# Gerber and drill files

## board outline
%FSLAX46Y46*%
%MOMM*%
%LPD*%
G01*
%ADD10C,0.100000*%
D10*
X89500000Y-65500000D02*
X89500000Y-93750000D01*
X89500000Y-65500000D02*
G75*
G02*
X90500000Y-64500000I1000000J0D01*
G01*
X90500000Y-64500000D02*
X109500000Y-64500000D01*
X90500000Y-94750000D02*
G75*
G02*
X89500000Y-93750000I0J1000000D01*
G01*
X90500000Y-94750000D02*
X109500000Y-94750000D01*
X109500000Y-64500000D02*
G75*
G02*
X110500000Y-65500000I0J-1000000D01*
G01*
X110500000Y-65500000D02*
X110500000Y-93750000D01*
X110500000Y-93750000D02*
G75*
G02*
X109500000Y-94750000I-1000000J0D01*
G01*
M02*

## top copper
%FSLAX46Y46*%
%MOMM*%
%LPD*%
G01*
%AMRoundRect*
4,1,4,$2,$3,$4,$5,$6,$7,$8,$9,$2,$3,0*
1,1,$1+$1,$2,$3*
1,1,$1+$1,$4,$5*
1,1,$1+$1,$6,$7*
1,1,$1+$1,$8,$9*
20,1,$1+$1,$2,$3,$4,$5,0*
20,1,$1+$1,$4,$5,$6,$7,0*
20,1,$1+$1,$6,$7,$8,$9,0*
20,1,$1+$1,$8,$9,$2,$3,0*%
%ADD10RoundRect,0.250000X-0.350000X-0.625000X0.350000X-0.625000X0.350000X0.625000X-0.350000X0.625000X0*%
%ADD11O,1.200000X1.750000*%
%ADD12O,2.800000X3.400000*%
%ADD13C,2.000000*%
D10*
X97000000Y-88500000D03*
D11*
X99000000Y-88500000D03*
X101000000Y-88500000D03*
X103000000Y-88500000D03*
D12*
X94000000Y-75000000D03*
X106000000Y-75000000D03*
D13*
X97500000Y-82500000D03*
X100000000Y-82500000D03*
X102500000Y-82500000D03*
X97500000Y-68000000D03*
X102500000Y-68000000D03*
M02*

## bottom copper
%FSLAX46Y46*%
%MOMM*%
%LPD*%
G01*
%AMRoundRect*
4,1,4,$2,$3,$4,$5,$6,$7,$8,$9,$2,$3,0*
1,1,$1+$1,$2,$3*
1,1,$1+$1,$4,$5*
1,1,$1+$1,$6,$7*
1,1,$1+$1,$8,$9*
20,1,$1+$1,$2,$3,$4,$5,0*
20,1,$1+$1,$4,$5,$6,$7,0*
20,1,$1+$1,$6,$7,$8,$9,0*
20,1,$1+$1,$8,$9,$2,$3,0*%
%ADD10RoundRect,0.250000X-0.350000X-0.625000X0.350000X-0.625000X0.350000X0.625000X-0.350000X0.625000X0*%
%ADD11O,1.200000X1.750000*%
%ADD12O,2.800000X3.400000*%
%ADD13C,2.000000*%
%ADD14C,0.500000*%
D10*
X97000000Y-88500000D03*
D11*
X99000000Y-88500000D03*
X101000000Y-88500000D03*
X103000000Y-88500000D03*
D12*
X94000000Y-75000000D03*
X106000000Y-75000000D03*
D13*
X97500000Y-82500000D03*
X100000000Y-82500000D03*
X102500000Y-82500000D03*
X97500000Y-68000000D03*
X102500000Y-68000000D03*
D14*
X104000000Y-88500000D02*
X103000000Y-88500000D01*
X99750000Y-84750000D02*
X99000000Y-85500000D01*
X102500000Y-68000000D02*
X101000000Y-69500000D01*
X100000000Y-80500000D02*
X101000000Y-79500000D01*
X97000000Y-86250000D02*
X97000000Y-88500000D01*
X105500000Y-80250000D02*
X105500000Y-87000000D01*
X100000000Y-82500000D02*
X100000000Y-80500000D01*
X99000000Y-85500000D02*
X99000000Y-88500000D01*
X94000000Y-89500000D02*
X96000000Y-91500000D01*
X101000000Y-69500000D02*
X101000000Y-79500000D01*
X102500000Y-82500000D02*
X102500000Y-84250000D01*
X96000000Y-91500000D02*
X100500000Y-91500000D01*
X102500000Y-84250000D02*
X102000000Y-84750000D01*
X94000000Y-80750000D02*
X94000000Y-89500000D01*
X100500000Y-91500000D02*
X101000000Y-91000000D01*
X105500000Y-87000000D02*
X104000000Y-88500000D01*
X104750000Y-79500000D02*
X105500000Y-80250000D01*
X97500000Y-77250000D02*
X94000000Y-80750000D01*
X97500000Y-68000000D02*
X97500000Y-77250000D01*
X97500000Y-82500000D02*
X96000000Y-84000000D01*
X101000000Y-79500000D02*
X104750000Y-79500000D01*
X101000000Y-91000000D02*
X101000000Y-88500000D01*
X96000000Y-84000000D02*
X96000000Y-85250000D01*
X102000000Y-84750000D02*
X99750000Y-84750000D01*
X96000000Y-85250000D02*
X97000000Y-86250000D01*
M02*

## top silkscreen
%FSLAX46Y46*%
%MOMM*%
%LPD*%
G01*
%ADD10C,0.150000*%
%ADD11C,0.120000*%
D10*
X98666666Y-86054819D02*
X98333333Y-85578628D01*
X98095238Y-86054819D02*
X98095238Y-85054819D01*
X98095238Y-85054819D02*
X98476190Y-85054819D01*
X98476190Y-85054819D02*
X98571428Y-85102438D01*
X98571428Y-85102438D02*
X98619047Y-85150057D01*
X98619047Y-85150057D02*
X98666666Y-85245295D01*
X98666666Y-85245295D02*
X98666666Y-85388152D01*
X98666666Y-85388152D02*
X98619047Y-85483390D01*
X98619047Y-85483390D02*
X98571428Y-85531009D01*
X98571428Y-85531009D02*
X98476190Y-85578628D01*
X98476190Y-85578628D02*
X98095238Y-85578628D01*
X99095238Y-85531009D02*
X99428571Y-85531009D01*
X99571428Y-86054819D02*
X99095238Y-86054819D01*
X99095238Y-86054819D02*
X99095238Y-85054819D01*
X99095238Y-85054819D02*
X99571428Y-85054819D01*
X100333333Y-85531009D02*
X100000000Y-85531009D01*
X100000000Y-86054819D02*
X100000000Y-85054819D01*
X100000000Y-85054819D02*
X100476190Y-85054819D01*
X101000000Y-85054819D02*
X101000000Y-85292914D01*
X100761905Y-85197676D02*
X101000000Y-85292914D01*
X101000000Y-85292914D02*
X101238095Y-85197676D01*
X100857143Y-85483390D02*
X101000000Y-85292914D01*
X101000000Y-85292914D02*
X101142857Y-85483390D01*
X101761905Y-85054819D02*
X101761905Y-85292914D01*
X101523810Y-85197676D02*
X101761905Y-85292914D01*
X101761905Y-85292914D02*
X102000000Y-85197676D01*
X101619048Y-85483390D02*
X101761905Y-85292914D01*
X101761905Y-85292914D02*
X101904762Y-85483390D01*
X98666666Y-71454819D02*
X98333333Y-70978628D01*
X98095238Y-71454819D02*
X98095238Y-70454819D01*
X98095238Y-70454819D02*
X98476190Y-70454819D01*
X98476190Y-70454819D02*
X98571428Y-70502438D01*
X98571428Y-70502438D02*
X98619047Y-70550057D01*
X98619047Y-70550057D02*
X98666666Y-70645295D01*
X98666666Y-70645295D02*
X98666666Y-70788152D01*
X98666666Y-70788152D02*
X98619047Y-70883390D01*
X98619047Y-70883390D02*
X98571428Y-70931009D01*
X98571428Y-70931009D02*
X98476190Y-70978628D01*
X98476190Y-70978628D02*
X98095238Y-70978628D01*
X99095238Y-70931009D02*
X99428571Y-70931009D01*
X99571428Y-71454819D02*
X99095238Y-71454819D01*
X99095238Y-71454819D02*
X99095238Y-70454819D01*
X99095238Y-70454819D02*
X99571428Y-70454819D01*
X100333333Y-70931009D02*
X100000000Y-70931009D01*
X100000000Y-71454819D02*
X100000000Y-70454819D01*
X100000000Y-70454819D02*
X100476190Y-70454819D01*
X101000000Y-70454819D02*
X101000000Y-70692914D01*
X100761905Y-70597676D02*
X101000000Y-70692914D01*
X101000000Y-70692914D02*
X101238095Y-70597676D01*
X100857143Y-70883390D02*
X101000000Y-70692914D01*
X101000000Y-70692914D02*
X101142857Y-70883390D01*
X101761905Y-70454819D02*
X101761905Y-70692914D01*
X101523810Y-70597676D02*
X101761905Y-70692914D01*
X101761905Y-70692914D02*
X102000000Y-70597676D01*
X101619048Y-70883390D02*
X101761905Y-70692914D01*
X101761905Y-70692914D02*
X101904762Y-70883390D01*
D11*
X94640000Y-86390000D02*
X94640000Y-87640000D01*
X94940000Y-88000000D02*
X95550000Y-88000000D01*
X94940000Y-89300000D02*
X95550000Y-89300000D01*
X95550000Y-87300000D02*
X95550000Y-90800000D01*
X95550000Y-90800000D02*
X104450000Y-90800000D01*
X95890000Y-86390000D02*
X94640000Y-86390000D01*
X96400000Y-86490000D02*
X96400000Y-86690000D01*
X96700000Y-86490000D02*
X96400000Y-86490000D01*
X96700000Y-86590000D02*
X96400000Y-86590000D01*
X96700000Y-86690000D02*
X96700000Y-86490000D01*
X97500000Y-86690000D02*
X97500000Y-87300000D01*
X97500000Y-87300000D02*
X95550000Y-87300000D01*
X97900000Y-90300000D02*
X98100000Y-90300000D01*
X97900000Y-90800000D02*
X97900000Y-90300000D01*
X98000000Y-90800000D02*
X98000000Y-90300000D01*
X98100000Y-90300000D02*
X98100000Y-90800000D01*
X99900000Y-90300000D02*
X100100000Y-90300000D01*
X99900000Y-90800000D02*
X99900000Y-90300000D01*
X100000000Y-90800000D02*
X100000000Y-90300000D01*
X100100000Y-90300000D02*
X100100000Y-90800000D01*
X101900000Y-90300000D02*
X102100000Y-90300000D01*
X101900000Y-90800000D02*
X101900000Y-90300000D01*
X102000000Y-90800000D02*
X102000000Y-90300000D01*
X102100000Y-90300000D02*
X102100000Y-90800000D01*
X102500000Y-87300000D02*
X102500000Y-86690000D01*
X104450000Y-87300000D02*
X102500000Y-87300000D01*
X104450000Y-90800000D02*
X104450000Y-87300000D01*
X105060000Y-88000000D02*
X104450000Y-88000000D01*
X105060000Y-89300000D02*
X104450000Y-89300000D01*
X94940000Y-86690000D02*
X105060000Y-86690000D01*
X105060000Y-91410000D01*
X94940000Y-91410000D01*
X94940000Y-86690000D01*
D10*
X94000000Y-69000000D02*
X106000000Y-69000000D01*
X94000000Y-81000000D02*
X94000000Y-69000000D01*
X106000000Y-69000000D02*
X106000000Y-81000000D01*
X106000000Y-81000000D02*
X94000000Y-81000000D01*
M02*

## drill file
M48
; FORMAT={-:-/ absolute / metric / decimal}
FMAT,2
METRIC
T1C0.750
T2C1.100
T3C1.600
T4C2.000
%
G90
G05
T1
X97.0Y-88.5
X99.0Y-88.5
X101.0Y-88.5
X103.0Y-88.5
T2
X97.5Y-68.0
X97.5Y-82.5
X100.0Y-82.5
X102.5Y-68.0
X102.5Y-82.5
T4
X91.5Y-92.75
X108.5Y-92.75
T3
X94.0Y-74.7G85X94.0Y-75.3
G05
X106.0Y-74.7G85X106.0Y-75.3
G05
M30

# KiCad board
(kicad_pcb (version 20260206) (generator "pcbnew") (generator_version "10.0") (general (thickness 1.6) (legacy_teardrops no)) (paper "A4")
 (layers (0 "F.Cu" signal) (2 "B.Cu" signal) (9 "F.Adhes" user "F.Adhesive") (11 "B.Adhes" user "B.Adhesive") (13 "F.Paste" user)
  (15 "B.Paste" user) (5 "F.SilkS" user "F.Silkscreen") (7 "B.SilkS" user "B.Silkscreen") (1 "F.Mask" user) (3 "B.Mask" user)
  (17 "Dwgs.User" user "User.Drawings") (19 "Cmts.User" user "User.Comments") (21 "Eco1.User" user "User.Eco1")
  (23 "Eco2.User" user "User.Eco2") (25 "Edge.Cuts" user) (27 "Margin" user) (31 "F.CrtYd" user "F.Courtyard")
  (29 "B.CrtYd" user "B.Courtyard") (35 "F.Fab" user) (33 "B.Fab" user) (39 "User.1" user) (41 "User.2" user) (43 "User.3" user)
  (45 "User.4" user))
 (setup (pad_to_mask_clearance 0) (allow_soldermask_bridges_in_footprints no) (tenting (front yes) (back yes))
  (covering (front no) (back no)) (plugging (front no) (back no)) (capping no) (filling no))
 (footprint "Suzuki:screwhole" (layer "F.Cu") (at 108.75 92.75)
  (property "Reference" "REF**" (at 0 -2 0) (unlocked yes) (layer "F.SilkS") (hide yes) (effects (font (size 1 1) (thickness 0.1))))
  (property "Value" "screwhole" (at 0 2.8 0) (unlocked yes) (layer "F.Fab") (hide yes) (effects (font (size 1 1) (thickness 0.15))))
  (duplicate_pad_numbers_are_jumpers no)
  (pad "" np_thru_hole circle (at -0.25 0) (size 2 2) (drill 2) (layers "*.Cu" "*.Mask")))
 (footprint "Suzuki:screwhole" (layer "F.Cu") (at 91.5 92.75)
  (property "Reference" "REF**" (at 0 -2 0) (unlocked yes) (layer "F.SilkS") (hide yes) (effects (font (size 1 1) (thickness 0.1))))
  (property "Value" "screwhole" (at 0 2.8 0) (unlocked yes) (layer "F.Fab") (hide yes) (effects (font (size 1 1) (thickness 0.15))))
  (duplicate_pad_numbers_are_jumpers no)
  (pad "" np_thru_hole circle (at 0 0) (size 2 2) (drill 2) (layers "*.Cu" "*.Mask")))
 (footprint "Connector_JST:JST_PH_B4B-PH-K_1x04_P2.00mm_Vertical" (layer "F.Cu") (at 97 88.5)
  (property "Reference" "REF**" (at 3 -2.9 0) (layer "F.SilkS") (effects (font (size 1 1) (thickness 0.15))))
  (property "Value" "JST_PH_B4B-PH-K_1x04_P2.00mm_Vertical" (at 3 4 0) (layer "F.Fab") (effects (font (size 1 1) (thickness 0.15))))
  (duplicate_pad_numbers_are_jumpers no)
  (fp_line (start -2.36 -2.11) (end -2.36 -0.86) (stroke (width 0.12) (type solid)) (layer "F.SilkS"))
  (fp_line (start -2.06 -0.5) (end -1.45 -0.5) (stroke (width 0.12) (type solid)) (layer "F.SilkS"))
  (fp_line (start -2.06 0.8) (end -1.45 0.8) (stroke (width 0.12) (type solid)) (layer "F.SilkS"))
  (fp_line (start -1.45 -1.2) (end -1.45 2.3) (stroke (width 0.12) (type solid)) (layer "F.SilkS"))
  (fp_line (start -1.45 2.3) (end 7.45 2.3) (stroke (width 0.12) (type solid)) (layer "F.SilkS"))
  (fp_line (start -1.11 -2.11) (end -2.36 -2.11) (stroke (width 0.12) (type solid)) (layer "F.SilkS"))
  (fp_line (start -0.6 -2.01) (end -0.6 -1.81) (stroke (width 0.12) (type solid)) (layer "F.SilkS"))
  (fp_line (start -0.3 -2.01) (end -0.6 -2.01) (stroke (width 0.12) (type solid)) (layer "F.SilkS"))
  (fp_line (start -0.3 -1.91) (end -0.6 -1.91) (stroke (width 0.12) (type solid)) (layer "F.SilkS"))
  (fp_line (start -0.3 -1.81) (end -0.3 -2.01) (stroke (width 0.12) (type solid)) (layer "F.SilkS"))
  (fp_line (start 0.5 -1.81) (end 0.5 -1.2) (stroke (width 0.12) (type solid)) (layer "F.SilkS"))
  (fp_line (start 0.5 -1.2) (end -1.45 -1.2) (stroke (width 0.12) (type solid)) (layer "F.SilkS"))
  (fp_line (start 0.9 1.8) (end 1.1 1.8) (stroke (width 0.12) (type solid)) (layer "F.SilkS"))
  (fp_line (start 0.9 2.3) (end 0.9 1.8) (stroke (width 0.12) (type solid)) (layer "F.SilkS"))
  (fp_line (start 1 2.3) (end 1 1.8) (stroke (width 0.12) (type solid)) (layer "F.SilkS"))
  (fp_line (start 1.1 1.8) (end 1.1 2.3) (stroke (width 0.12) (type solid)) (layer "F.SilkS"))
  (fp_line (start 2.9 1.8) (end 3.1 1.8) (stroke (width 0.12) (type solid)) (layer "F.SilkS"))
  (fp_line (start 2.9 2.3) (end 2.9 1.8) (stroke (width 0.12) (type solid)) (layer "F.SilkS"))
  (fp_line (start 3 2.3) (end 3 1.8) (stroke (width 0.12) (type solid)) (layer "F.SilkS"))
  (fp_line (start 3.1 1.8) (end 3.1 2.3) (stroke (width 0.12) (type solid)) (layer "F.SilkS"))
  (fp_line (start 4.9 1.8) (end 5.1 1.8) (stroke (width 0.12) (type solid)) (layer "F.SilkS"))
  (fp_line (start 4.9 2.3) (end 4.9 1.8) (stroke (width 0.12) (type solid)) (layer "F.SilkS"))
  (fp_line (start 5 2.3) (end 5 1.8) (stroke (width 0.12) (type solid)) (layer "F.SilkS"))
  (fp_line (start 5.1 1.8) (end 5.1 2.3) (stroke (width 0.12) (type solid)) (layer "F.SilkS"))
  (fp_line (start 5.5 -1.2) (end 5.5 -1.81) (stroke (width 0.12) (type solid)) (layer "F.SilkS"))
  (fp_line (start 7.45 -1.2) (end 5.5 -1.2) (stroke (width 0.12) (type solid)) (layer "F.SilkS"))
  (fp_line (start 7.45 2.3) (end 7.45 -1.2) (stroke (width 0.12) (type solid)) (layer "F.SilkS"))
  (fp_line (start 8.06 -0.5) (end 7.45 -0.5) (stroke (width 0.12) (type solid)) (layer "F.SilkS"))
  (fp_line (start 8.06 0.8) (end 7.45 0.8) (stroke (width 0.12) (type solid)) (layer "F.SilkS"))
  (fp_rect (start -2.06 -1.81) (end 8.06 2.91) (stroke (width 0.12) (type solid)) (fill no) (layer "F.SilkS"))
  (pad "1" thru_hole roundrect (at 0 0) (size 1.2 1.75) (drill 0.75) (layers "*.Cu" "*.Mask") (remove_unused_layers no)
   (roundrect_rratio 0.208333))
  (pad "2" thru_hole oval (at 2 0) (size 1.2 1.75) (drill 0.75) (layers "*.Cu" "*.Mask") (remove_unused_layers no))
  (pad "3" thru_hole oval (at 4 0) (size 1.2 1.75) (drill 0.75) (layers "*.Cu" "*.Mask") (remove_unused_layers no))
  (pad "4" thru_hole oval (at 6 0) (size 1.2 1.75) (drill 0.75) (layers "*.Cu" "*.Mask") (remove_unused_layers no)))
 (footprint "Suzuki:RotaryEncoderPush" (layer "F.Cu") (at 100 75)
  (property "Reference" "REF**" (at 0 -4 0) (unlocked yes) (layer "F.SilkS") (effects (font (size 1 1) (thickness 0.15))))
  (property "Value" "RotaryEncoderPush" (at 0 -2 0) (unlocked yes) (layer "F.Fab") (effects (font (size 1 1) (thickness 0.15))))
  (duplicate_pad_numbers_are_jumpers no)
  (fp_line (start -6 -6) (end 6 -6) (stroke (width 0.15) (type solid)) (layer "F.SilkS"))
  (fp_line (start -6 6) (end -6 -6) (stroke (width 0.15) (type solid)) (layer "F.SilkS"))
  (fp_line (start 6 -6) (end 6 6) (stroke (width 0.15) (type solid)) (layer "F.SilkS"))
  (fp_line (start 6 6) (end -6 6) (stroke (width 0.15) (type solid)) (layer "F.SilkS"))
  (pad "" thru_hole oval (at -6 0) (size 2.8 3.4) (drill oval 1.6 2.2) (layers "*.Cu" "*.Mask") (remove_unused_layers no)
   (thermal_bridge_angle 45))
  (pad "" thru_hole oval (at 6 0) (size 2.8 3.4) (drill oval 1.6 2.2) (layers "*.Cu" "*.Mask") (remove_unused_layers no)
   (thermal_bridge_angle 45))
  (pad "1" thru_hole circle (at -2.5 7.5) (size 2 2) (drill 1.1) (layers "*.Cu" "*.Mask") (remove_unused_layers no))
  (pad "2" thru_hole circle (at 0 7.5) (size 2 2) (drill 1.1) (layers "*.Cu" "*.Mask") (remove_unused_layers no))
  (pad "3" thru_hole circle (at 2.5 7.5) (size 2 2) (drill 1.1) (layers "*.Cu" "*.Mask") (remove_unused_layers no))
  (pad "4" thru_hole circle (at -2.5 -7) (size 2 2) (drill 1.1) (layers "*.Cu" "*.Mask") (remove_unused_layers no))
  (pad "5" thru_hole circle (at 2.5 -7) (size 2 2) (drill 1.1) (layers "*.Cu" "*.Mask") (remove_unused_layers no)))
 (gr_line (start 89.5 65.5) (end 89.5 93.75) (stroke (width 0.1) (type solid)) (layer "Edge.Cuts"))
 (gr_arc (start 89.5 65.5) (mid 89.792893 64.792893) (end 90.5 64.5) (stroke (width 0.1) (type default)) (layer "Edge.Cuts"))
 (gr_line (start 90.5 64.5) (end 109.5 64.5) (stroke (width 0.1) (type solid)) (layer "Edge.Cuts"))
 (gr_arc (start 90.5 94.75) (mid 89.792893 94.457107) (end 89.5 93.75) (stroke (width 0.1) (type default)) (layer "Edge.Cuts"))
 (gr_line (start 90.5 94.75) (end 109.5 94.75) (stroke (width 0.1) (type solid)) (layer "Edge.Cuts"))
 (gr_arc (start 109.5 64.5) (mid 110.207107 64.792893) (end 110.5 65.5) (stroke (width 0.1) (type default)) (layer "Edge.Cuts"))
 (gr_line (start 110.5 65.5) (end 110.5 93.75) (stroke (width 0.1) (type solid)) (layer "Edge.Cuts"))
 (gr_arc (start 110.5 93.75) (mid 110.207107 94.457107) (end 109.5 94.75) (stroke (width 0.1) (type default)) (layer "Edge.Cuts"))
 (segment (start 104 88.5) (end 103 88.5) (width 0.5) (layer "B.Cu") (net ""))
 (segment (start 99.75 84.75) (end 99 85.5) (width 0.5) (layer "B.Cu") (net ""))
 (segment (start 102.5 68) (end 101 69.5) (width 0.5) (layer "B.Cu") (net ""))
 (segment (start 100 80.5) (end 101 79.5) (width 0.5) (layer "B.Cu") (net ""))
 (segment (start 97 86.25) (end 97 88.5) (width 0.5) (layer "B.Cu") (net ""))
 (segment (start 105.5 80.25) (end 105.5 87) (width 0.5) (layer "B.Cu") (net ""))
 (segment (start 100 82.5) (end 100 80.5) (width 0.5) (layer "B.Cu") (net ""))
 (segment (start 99 85.5) (end 99 88.5) (width 0.5) (layer "B.Cu") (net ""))
 (segment (start 94 89.5) (end 96 91.5) (width 0.5) (layer "B.Cu") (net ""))
 (segment (start 101 69.5) (end 101 79.5) (width 0.5) (layer "B.Cu") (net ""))
 (segment (start 102.5 82.5) (end 102.5 84.25) (width 0.5) (layer "B.Cu") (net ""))
 (segment (start 96 91.5) (end 100.5 91.5) (width 0.5) (layer "B.Cu") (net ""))
 (segment (start 102.5 84.25) (end 102 84.75) (width 0.5) (layer "B.Cu") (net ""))
 (segment (start 94 80.75) (end 94 89.5) (width 0.5) (layer "B.Cu") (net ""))
 (segment (start 100.5 91.5) (end 101 91) (width 0.5) (layer "B.Cu") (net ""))
 (segment (start 105.5 87) (end 104 88.5) (width 0.5) (layer "B.Cu") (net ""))
 (segment (start 104.75 79.5) (end 105.5 80.25) (width 0.5) (layer "B.Cu") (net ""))
 (segment (start 97.5 77.25) (end 94 80.75) (width 0.5) (layer "B.Cu") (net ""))
 (segment (start 97.5 68) (end 97.5 77.25) (width 0.5) (layer "B.Cu") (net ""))
 (segment (start 97.5 82.5) (end 96 84) (width 0.5) (layer "B.Cu") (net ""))
 (segment (start 101 79.5) (end 104.75 79.5) (width 0.5) (layer "B.Cu") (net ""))
 (segment (start 101 91) (end 101 88.5) (width 0.5) (layer "B.Cu") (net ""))
 (segment (start 96 84) (end 96 85.25) (width 0.5) (layer "B.Cu") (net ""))
 (segment (start 102 84.75) (end 99.75 84.75) (width 0.5) (layer "B.Cu") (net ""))
 (segment (start 96 85.25) (end 97 86.25) (width 0.5) (layer "B.Cu") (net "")))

